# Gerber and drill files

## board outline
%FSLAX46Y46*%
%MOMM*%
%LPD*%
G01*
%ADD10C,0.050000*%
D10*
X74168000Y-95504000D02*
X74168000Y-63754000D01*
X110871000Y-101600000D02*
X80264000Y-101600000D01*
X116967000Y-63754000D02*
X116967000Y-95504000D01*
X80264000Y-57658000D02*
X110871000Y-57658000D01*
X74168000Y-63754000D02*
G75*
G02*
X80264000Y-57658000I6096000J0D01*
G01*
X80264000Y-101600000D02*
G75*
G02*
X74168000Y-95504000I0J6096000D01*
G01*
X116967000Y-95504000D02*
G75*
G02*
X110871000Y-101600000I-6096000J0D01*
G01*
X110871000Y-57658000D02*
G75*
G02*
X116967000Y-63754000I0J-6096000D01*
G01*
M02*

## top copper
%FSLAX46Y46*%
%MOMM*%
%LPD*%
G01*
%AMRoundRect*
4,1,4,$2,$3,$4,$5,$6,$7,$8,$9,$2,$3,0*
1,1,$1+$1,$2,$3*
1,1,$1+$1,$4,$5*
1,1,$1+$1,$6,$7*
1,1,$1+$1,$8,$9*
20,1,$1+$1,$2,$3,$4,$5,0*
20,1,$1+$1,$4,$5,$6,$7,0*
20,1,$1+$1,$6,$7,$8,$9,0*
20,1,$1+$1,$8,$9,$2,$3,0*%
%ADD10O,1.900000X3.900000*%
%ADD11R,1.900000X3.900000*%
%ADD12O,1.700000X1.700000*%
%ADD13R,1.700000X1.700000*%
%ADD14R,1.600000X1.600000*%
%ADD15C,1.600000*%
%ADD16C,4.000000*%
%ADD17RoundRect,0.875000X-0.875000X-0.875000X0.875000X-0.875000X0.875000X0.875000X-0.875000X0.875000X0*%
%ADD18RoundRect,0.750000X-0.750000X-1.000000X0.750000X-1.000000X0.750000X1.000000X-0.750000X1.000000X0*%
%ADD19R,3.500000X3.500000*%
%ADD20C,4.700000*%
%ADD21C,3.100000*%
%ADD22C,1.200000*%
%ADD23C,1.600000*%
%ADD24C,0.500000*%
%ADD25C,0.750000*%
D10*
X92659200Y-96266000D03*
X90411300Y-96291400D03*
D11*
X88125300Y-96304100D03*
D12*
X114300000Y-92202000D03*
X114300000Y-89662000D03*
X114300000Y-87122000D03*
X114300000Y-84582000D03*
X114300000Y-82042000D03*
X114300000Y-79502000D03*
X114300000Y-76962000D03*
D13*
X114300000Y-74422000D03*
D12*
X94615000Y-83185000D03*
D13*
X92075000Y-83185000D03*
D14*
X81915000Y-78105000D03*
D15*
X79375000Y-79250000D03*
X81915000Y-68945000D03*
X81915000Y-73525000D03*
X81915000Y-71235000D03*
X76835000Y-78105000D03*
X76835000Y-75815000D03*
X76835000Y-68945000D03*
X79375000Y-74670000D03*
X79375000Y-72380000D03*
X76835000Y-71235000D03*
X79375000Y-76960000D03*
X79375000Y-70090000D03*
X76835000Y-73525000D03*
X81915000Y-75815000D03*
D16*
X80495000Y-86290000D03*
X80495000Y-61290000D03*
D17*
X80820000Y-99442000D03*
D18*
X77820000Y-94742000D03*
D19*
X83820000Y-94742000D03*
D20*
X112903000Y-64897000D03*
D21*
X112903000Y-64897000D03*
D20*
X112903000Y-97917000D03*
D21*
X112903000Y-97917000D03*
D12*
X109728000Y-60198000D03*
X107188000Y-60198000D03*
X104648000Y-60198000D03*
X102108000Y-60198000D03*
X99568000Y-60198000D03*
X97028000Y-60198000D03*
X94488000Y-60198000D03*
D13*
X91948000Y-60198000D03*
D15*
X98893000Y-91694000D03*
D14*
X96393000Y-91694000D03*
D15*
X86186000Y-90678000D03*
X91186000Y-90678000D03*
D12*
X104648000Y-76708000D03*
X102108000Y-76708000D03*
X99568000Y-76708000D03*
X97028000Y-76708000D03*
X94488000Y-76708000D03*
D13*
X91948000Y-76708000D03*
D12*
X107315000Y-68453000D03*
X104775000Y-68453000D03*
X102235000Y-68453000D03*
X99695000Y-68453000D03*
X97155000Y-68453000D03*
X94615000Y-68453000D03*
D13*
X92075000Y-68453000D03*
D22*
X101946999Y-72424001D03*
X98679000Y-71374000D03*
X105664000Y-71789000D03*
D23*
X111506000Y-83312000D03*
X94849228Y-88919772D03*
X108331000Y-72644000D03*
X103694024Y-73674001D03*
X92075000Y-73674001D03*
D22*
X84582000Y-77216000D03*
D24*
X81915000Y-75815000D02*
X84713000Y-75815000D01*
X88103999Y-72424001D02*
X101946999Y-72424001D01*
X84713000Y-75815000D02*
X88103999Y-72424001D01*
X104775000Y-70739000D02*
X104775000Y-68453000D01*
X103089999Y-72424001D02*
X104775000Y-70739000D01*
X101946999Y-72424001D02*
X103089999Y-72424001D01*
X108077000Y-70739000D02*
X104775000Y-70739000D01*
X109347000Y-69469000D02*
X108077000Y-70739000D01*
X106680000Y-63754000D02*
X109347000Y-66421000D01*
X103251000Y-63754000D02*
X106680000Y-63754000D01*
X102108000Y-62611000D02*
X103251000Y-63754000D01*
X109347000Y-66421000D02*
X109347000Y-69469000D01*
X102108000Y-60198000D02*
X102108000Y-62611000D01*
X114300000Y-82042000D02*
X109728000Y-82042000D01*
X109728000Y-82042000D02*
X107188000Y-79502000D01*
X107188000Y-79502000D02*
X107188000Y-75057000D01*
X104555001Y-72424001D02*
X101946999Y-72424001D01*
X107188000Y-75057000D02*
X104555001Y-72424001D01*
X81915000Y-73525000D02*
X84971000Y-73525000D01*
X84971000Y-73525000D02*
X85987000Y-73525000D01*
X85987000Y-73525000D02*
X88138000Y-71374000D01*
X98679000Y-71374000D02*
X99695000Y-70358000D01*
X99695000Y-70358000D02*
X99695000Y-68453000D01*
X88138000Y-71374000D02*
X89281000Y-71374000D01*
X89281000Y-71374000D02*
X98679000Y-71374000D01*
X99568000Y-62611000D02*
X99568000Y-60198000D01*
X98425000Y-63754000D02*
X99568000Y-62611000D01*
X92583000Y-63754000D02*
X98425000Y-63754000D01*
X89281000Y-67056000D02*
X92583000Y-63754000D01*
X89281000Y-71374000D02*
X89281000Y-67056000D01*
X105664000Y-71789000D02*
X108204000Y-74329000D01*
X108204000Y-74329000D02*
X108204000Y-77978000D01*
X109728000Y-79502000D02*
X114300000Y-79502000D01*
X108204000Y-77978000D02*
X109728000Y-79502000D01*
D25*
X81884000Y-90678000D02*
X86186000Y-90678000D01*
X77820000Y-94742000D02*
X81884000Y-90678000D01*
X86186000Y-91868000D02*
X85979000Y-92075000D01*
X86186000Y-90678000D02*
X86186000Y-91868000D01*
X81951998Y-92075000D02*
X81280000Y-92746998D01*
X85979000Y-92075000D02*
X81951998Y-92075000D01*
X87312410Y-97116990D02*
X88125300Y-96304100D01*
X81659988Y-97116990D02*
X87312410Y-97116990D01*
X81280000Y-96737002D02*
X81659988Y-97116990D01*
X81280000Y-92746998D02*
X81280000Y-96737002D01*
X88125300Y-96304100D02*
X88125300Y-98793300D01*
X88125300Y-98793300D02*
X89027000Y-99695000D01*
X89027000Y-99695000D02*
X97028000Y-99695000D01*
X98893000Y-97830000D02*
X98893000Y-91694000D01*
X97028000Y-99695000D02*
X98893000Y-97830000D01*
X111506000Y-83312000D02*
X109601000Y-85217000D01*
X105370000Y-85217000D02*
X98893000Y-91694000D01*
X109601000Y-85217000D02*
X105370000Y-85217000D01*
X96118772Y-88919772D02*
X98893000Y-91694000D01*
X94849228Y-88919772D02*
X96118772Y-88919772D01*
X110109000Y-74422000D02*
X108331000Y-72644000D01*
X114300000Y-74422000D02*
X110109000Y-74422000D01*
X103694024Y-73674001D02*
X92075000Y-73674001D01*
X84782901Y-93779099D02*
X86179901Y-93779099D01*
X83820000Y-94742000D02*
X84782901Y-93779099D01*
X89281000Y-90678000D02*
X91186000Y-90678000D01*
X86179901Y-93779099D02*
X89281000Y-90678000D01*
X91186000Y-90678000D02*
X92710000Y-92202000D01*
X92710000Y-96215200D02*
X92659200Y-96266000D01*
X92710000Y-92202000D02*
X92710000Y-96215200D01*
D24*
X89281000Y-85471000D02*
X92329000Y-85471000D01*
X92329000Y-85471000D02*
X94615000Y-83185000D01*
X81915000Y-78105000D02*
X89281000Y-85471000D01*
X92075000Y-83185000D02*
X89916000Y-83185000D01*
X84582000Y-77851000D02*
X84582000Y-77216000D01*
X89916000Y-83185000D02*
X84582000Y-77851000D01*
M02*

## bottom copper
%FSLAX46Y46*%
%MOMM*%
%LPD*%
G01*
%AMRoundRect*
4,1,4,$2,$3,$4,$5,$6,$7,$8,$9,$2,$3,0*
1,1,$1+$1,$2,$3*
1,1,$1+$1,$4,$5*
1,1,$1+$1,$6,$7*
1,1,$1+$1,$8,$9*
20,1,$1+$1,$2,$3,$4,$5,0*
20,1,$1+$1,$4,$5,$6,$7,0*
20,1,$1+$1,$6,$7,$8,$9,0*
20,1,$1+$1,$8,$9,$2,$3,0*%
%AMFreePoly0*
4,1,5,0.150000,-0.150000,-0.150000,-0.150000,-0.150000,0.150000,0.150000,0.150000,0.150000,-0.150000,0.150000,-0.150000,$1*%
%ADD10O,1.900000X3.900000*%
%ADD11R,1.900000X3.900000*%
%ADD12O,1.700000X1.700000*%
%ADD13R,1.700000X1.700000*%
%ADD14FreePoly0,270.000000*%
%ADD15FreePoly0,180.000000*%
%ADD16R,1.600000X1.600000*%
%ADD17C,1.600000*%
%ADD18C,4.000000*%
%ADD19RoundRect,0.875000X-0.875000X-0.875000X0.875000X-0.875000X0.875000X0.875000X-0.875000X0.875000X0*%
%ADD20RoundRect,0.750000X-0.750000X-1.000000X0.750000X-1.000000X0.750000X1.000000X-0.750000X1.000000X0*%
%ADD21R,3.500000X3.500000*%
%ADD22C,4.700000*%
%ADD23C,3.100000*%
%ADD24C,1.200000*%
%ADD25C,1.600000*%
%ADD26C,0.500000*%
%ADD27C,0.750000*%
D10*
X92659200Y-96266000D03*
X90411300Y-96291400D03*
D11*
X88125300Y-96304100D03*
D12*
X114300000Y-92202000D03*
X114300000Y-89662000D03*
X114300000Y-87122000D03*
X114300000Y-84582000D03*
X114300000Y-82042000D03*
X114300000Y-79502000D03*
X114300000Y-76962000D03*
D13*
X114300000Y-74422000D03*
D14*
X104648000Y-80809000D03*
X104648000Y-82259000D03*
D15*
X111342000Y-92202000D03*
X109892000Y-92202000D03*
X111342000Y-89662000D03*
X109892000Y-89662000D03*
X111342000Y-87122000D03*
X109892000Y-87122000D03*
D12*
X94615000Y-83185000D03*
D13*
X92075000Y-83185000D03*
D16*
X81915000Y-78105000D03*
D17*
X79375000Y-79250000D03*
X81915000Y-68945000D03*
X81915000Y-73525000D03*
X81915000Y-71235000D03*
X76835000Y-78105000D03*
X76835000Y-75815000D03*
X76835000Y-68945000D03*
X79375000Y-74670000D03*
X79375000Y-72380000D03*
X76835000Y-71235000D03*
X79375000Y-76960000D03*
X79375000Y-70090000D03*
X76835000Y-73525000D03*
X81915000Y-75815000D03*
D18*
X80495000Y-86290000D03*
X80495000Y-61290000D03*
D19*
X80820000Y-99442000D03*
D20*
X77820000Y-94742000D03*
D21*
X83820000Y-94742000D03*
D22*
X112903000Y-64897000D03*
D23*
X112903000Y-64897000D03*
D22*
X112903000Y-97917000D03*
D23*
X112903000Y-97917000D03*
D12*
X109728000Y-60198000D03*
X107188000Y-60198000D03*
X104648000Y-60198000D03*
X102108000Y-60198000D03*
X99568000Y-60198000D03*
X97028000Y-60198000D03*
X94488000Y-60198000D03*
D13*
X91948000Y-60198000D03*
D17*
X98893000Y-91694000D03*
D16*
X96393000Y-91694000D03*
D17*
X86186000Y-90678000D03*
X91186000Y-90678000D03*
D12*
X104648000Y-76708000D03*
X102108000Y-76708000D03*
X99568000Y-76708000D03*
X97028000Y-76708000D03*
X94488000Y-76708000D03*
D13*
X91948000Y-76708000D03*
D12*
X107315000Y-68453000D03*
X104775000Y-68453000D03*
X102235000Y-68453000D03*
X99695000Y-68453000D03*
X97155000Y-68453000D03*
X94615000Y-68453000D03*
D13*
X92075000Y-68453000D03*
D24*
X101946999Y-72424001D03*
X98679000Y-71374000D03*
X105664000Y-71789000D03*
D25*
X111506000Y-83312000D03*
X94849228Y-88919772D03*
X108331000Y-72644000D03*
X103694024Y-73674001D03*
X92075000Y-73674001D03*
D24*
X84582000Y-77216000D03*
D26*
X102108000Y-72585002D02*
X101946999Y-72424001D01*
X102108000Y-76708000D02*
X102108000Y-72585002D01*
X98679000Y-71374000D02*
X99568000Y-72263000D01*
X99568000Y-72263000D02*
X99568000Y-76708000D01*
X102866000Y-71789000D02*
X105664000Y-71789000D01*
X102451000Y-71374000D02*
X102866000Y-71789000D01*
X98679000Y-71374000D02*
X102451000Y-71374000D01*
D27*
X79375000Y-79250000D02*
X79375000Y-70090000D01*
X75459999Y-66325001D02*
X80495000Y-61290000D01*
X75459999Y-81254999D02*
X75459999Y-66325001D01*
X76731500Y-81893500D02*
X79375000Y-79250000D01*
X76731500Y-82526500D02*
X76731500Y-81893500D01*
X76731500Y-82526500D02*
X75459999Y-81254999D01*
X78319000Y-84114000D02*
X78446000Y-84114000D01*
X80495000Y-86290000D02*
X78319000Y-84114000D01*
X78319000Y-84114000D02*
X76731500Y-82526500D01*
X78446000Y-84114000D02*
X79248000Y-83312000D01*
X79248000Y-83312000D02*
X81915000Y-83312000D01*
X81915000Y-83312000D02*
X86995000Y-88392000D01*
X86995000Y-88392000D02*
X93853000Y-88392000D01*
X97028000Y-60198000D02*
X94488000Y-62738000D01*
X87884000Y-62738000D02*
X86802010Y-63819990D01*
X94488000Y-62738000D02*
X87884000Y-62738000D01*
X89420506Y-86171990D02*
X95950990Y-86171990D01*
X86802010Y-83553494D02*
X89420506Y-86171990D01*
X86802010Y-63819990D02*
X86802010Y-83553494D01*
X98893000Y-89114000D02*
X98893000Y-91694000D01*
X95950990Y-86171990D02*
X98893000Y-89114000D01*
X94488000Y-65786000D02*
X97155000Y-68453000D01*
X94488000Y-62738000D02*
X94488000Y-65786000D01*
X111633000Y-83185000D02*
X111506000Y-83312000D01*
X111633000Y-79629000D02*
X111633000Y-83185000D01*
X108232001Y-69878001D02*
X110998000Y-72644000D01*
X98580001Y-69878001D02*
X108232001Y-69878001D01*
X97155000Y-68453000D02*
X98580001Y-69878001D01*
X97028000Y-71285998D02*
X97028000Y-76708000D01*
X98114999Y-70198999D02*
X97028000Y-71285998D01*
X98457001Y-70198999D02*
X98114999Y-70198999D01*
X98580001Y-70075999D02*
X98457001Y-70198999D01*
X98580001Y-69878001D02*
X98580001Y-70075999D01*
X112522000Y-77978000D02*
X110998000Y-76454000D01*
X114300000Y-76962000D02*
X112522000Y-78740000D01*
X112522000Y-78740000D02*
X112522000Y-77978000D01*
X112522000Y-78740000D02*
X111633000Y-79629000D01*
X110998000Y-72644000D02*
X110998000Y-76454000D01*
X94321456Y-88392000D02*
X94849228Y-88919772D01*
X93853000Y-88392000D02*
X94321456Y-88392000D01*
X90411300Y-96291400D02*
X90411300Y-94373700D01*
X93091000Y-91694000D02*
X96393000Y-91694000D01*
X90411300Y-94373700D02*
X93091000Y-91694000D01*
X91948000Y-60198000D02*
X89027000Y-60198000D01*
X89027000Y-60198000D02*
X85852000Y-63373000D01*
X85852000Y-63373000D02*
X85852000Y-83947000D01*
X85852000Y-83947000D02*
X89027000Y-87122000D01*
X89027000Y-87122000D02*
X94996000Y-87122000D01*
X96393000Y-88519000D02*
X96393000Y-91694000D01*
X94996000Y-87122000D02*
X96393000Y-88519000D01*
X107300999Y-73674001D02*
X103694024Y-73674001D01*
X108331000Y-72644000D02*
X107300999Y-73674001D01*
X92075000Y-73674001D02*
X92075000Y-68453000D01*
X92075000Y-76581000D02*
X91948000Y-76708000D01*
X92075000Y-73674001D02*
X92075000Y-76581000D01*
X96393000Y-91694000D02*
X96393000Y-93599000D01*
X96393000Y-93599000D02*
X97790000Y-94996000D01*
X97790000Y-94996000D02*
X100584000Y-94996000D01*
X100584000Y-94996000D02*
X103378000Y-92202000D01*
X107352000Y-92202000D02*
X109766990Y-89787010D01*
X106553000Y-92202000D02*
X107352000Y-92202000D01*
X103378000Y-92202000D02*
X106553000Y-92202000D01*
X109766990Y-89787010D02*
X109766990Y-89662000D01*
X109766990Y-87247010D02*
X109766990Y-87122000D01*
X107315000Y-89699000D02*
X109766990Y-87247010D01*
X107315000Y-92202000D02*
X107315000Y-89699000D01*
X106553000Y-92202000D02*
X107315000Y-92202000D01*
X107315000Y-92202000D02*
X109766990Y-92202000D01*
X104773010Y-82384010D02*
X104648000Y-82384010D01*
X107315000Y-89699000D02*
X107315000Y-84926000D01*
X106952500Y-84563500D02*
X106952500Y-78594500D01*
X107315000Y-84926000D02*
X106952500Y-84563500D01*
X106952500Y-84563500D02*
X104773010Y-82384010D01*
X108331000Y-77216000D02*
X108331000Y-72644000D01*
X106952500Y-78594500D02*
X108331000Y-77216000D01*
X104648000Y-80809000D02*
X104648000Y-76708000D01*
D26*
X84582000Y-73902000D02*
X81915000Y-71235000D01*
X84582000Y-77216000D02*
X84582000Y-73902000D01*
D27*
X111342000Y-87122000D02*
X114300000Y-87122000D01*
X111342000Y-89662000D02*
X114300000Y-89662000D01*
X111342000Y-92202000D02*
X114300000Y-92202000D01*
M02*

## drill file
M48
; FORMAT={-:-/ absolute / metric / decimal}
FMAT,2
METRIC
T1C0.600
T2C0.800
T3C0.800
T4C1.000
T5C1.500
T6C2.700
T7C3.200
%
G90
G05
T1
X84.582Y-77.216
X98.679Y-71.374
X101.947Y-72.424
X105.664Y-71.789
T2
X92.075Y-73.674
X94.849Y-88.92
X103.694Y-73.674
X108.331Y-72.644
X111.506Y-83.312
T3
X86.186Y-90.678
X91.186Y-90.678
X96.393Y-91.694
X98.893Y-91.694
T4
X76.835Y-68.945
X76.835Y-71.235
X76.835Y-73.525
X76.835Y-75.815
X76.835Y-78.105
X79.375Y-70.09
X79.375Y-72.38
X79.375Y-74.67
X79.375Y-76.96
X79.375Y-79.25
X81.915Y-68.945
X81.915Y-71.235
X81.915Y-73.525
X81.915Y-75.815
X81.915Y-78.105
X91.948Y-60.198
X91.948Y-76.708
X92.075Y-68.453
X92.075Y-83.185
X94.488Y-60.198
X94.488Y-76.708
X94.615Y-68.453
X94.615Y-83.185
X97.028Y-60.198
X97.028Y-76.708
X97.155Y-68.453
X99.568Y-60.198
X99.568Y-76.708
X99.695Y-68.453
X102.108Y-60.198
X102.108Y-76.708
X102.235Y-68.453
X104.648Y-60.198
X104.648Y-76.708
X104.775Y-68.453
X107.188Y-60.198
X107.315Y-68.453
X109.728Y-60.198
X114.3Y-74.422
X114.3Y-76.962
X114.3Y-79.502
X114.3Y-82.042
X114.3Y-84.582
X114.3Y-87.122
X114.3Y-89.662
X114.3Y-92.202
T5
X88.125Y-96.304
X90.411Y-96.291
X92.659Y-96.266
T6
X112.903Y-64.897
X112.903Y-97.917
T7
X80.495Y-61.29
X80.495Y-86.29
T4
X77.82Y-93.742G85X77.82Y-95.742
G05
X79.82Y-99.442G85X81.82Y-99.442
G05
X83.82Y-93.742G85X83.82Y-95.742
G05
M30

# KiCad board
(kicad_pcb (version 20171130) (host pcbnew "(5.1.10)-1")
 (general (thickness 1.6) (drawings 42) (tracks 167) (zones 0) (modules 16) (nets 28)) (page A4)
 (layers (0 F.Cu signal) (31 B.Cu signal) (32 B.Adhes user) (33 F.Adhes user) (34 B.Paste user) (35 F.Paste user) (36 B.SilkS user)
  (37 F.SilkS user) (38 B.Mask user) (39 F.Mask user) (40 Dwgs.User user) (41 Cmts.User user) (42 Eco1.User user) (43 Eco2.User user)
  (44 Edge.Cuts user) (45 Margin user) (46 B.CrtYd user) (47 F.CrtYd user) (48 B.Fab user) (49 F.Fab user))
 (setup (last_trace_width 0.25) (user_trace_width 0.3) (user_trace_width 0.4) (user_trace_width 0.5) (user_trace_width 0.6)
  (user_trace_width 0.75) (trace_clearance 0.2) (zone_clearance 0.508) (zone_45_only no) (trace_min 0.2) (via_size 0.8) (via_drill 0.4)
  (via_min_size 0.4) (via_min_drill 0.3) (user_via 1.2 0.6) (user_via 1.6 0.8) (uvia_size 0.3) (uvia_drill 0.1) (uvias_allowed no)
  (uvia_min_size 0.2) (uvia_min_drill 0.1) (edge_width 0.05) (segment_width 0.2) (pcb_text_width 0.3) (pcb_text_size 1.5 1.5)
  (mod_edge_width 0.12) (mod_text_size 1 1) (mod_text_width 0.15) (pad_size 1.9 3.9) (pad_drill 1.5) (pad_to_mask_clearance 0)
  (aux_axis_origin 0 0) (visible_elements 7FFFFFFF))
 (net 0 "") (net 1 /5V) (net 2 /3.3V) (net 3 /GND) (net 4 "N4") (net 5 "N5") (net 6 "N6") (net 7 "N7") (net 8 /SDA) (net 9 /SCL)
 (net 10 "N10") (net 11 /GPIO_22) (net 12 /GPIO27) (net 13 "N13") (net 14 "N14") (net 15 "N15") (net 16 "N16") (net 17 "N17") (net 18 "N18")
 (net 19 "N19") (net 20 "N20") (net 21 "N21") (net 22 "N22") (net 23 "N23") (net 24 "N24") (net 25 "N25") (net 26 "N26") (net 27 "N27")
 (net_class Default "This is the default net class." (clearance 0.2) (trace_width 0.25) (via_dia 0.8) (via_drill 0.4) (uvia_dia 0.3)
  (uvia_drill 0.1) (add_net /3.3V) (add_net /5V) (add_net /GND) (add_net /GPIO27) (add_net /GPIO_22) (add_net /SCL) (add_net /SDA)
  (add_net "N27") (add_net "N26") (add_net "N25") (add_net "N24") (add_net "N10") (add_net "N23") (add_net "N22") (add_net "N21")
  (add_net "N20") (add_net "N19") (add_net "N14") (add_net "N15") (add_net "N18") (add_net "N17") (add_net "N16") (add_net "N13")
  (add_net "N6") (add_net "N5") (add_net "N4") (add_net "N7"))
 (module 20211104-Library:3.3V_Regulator (layer F.Cu) (at 84.963 96.266)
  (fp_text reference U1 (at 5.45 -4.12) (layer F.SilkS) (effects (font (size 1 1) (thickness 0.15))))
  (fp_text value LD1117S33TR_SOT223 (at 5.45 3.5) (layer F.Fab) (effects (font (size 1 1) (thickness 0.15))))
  (pad 3 thru_hole oval (at 7.6962 0) (size 1.9 3.9) (drill 1.5) (layers *.Cu *.Mask) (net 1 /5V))
  (pad 2 thru_hole oval (at 5.4483 0.0254) (size 1.9 3.9) (drill 1.5) (layers *.Cu *.Mask) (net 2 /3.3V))
  (pad 1 thru_hole rect (at 3.1623 0.0381) (size 1.9 3.9) (drill 1.5) (layers *.Cu *.Mask) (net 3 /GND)))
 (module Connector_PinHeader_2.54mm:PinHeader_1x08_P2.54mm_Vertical (layer F.Cu) (at 114.3 74.422)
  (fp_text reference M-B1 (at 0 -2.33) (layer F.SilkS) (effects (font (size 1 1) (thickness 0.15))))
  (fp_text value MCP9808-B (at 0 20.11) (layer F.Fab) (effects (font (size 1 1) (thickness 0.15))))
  (pad 8 thru_hole oval (at 0 17.78) (size 1.7 1.7) (drill 1) (layers *.Cu *.Mask) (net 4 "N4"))
  (pad 7 thru_hole oval (at 0 15.24) (size 1.7 1.7) (drill 1) (layers *.Cu *.Mask) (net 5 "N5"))
  (pad 6 thru_hole oval (at 0 12.7) (size 1.7 1.7) (drill 1) (layers *.Cu *.Mask) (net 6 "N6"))
  (pad 5 thru_hole oval (at 0 10.16) (size 1.7 1.7) (drill 1) (layers *.Cu *.Mask) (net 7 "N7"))
  (pad 4 thru_hole oval (at 0 7.62) (size 1.7 1.7) (drill 1) (layers *.Cu *.Mask) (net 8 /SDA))
  (pad 3 thru_hole oval (at 0 5.08) (size 1.7 1.7) (drill 1) (layers *.Cu *.Mask) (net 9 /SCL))
  (pad 2 thru_hole oval (at 0 2.54) (size 1.7 1.7) (drill 1) (layers *.Cu *.Mask) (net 3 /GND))
  (pad 1 thru_hole rect (at 0 0) (size 1.7 1.7) (drill 1) (layers *.Cu *.Mask) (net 2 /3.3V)))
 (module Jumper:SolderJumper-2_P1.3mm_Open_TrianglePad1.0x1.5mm (layer B.Cu) (at 104.648 81.534 270)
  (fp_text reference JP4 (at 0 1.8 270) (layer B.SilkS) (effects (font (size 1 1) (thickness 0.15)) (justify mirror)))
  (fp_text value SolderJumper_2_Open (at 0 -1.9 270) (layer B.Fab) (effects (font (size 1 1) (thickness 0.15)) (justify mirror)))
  (pad 1 smd custom (at -0.725 0 270) (size 0.3 0.3) (layers B.Cu B.Mask) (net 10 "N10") (zone_connect 2)
   (options (clearance outline) (anchor rect)) (primitives))
  (pad 2 smd custom (at 0.725 0 270) (size 0.3 0.3) (layers B.Cu B.Mask) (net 2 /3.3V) (zone_connect 2)
   (options (clearance outline) (anchor rect)) (primitives)))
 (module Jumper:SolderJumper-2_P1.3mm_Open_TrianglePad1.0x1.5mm (layer B.Cu) (at 110.617 92.202 180)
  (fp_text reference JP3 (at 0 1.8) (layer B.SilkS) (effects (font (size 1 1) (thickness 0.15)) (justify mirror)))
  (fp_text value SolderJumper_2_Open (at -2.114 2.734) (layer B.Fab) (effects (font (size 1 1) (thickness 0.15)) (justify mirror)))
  (pad 1 smd custom (at -0.725 0 180) (size 0.3 0.3) (layers B.Cu B.Mask) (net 4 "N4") (zone_connect 2)
   (options (clearance outline) (anchor rect)) (primitives))
  (pad 2 smd custom (at 0.725 0 180) (size 0.3 0.3) (layers B.Cu B.Mask) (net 2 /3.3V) (zone_connect 2)
   (options (clearance outline) (anchor rect)) (primitives)))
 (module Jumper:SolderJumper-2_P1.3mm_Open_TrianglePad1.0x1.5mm (layer B.Cu) (at 110.617 89.662 180)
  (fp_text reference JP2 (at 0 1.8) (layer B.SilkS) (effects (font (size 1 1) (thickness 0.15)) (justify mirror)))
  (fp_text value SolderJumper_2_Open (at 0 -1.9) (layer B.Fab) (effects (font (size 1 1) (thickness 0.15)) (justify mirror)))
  (pad 1 smd custom (at -0.725 0 180) (size 0.3 0.3) (layers B.Cu B.Mask) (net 5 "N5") (zone_connect 2)
   (options (clearance outline) (anchor rect)) (primitives))
  (pad 2 smd custom (at 0.725 0 180) (size 0.3 0.3) (layers B.Cu B.Mask) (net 2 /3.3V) (zone_connect 2)
   (options (clearance outline) (anchor rect)) (primitives)))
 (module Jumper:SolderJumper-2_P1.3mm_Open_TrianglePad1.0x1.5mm (layer B.Cu) (at 110.617 87.122 180)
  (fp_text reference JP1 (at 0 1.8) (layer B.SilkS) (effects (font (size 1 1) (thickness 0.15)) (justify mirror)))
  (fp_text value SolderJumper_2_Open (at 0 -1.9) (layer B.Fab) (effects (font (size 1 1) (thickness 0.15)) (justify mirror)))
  (pad 1 smd custom (at -0.725 0 180) (size 0.3 0.3) (layers B.Cu B.Mask) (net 6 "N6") (zone_connect 2)
   (options (clearance outline) (anchor rect)) (primitives))
  (pad 2 smd custom (at 0.725 0 180) (size 0.3 0.3) (layers B.Cu B.Mask) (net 2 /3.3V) (zone_connect 2)
   (options (clearance outline) (anchor rect)) (primitives)))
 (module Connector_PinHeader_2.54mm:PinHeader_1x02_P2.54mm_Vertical (layer F.Cu) (at 92.075 83.185 90)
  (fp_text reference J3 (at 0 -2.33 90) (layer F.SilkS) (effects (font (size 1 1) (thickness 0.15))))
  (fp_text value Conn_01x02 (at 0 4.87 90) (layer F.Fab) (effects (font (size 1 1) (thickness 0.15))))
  (pad 2 thru_hole oval (at 0 2.54 90) (size 1.7 1.7) (drill 1) (layers *.Cu *.Mask) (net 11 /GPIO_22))
  (pad 1 thru_hole rect (at 0 0 90) (size 1.7 1.7) (drill 1) (layers *.Cu *.Mask) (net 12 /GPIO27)))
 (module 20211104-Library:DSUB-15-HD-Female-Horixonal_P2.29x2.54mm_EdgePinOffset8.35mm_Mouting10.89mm (layer F.Cu) (at 81.915 78.105 270)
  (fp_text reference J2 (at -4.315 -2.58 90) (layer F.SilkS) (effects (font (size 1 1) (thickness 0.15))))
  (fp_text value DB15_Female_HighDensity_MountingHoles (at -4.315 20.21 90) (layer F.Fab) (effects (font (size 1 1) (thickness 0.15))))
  (pad 1 thru_hole rect (at 0 0 270) (size 1.6 1.6) (drill 1) (layers *.Cu *.Mask) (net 11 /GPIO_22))
  (pad 6 thru_hole circle (at 1.145 2.54 270) (size 1.6 1.6) (drill 1) (layers *.Cu *.Mask) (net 3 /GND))
  (pad 5 thru_hole circle (at -9.16 0 270) (size 1.6 1.6) (drill 1) (layers *.Cu *.Mask) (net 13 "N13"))
  (pad 3 thru_hole circle (at -4.58 0 270) (size 1.6 1.6) (drill 1) (layers *.Cu *.Mask) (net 9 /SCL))
  (pad 4 thru_hole circle (at -6.87 0 270) (size 1.6 1.6) (drill 1) (layers *.Cu *.Mask) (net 12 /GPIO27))
  (pad 11 thru_hole circle (at 0 5.08 270) (size 1.6 1.6) (drill 1) (layers *.Cu *.Mask) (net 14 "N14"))
  (pad 12 thru_hole circle (at -2.29 5.08 270) (size 1.6 1.6) (drill 1) (layers *.Cu *.Mask) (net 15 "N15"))
  (pad 15 thru_hole circle (at -9.16 5.08 270) (size 1.6 1.6) (drill 1) (layers *.Cu *.Mask) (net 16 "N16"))
  (pad 8 thru_hole circle (at -3.435 2.54 270) (size 1.6 1.6) (drill 1) (layers *.Cu *.Mask) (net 3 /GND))
  (pad 9 thru_hole circle (at -5.725 2.54 270) (size 1.6 1.6) (drill 1) (layers *.Cu *.Mask) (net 3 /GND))
  (pad 14 thru_hole circle (at -6.87 5.08 270) (size 1.6 1.6) (drill 1) (layers *.Cu *.Mask) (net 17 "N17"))
  (pad 7 thru_hole circle (at -1.145 2.54 270) (size 1.6 1.6) (drill 1) (layers *.Cu *.Mask) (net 3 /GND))
  (pad 10 thru_hole circle (at -8.015 2.54 270) (size 1.6 1.6) (drill 1) (layers *.Cu *.Mask) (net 3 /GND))
  (pad 13 thru_hole circle (at -4.58 5.08 270) (size 1.6 1.6) (drill 1) (layers *.Cu *.Mask) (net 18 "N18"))
  (pad 2 thru_hole circle (at -2.29 0 270) (size 1.6 1.6) (drill 1) (layers *.Cu *.Mask) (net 8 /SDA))
  (pad 0 thru_hole circle (at 8.185 1.42 270) (size 4 4) (drill 3.2) (layers *.Cu *.Mask) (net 3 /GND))
  (pad 0 thru_hole circle (at -16.815 1.42 270) (size 4 4) (drill 3.2) (layers *.Cu *.Mask) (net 3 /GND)))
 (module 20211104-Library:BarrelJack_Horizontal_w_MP (layer F.Cu) (at 83.82 94.742)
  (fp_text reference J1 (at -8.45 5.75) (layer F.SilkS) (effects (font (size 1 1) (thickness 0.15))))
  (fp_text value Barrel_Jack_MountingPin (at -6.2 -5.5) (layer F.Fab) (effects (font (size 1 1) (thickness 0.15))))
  (pad MP thru_hole roundrect (at -3 4.7) (size 3.5 3.5) (drill oval 3 1) (layers *.Cu *.Mask) (roundrect_rratio 0.25) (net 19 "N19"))
  (pad 2 thru_hole roundrect (at -6 0) (size 3 3.5) (drill oval 1 3) (layers *.Cu *.Mask) (roundrect_rratio 0.25) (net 3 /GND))
  (pad 1 thru_hole rect (at 0 0) (size 3.5 3.5) (drill oval 1 3) (layers *.Cu *.Mask) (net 1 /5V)))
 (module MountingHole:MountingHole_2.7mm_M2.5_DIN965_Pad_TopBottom (layer F.Cu) (at 112.903 64.897)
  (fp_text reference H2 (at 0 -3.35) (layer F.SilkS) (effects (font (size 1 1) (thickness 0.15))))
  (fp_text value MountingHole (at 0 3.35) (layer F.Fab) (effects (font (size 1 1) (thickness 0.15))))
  (pad 1 connect circle (at 0 0) (size 4.7 4.7) (layers B.Cu B.Mask))
  (pad 1 connect circle (at 0 0) (size 4.7 4.7) (layers F.Cu F.Mask))
  (pad 1 thru_hole circle (at 0 0) (size 3.1 3.1) (drill 2.7) (layers *.Cu *.Mask)))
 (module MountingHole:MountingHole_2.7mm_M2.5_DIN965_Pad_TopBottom (layer F.Cu) (at 112.903 97.917)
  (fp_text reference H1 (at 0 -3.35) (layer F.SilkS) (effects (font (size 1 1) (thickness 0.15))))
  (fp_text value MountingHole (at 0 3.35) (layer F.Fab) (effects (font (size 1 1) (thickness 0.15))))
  (pad 1 connect circle (at 0 0) (size 4.7 4.7) (layers B.Cu B.Mask))
  (pad 1 connect circle (at 0 0) (size 4.7 4.7) (layers F.Cu F.Mask))
  (pad 1 thru_hole circle (at 0 0) (size 3.1 3.1) (drill 2.7) (layers *.Cu *.Mask)))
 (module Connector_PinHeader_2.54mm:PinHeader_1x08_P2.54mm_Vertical (layer F.Cu) (at 91.948 60.198 90)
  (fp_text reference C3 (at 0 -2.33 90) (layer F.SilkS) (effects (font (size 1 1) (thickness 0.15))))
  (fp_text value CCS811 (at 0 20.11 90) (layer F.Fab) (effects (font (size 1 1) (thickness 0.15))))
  (pad 8 thru_hole oval (at 0 17.78 90) (size 1.7 1.7) (drill 1) (layers *.Cu *.Mask) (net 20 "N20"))
  (pad 7 thru_hole oval (at 0 15.24 90) (size 1.7 1.7) (drill 1) (layers *.Cu *.Mask) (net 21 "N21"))
  (pad 6 thru_hole oval (at 0 12.7 90) (size 1.7 1.7) (drill 1) (layers *.Cu *.Mask) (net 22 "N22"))
  (pad 5 thru_hole oval (at 0 10.16 90) (size 1.7 1.7) (drill 1) (layers *.Cu *.Mask) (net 8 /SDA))
  (pad 4 thru_hole oval (at 0 7.62 90) (size 1.7 1.7) (drill 1) (layers *.Cu *.Mask) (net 9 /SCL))
  (pad 3 thru_hole oval (at 0 5.08 90) (size 1.7 1.7) (drill 1) (layers *.Cu *.Mask) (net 3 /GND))
  (pad 2 thru_hole oval (at 0 2.54 90) (size 1.7 1.7) (drill 1) (layers *.Cu *.Mask) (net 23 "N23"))
  (pad 1 thru_hole rect (at 0 0 90) (size 1.7 1.7) (drill 1) (layers *.Cu *.Mask) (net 2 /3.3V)))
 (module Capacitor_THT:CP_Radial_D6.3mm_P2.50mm (layer F.Cu) (at 96.393 91.694)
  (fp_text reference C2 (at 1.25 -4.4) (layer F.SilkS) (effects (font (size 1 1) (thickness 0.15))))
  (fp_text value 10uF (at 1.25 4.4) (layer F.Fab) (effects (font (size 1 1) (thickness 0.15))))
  (pad 2 thru_hole circle (at 2.5 0) (size 1.6 1.6) (drill 0.8) (layers *.Cu *.Mask) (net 3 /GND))
  (pad 1 thru_hole rect (at 0 0) (size 1.6 1.6) (drill 0.8) (layers *.Cu *.Mask) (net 2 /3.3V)))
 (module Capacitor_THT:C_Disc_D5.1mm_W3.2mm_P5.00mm (layer F.Cu) (at 91.186 90.678 180)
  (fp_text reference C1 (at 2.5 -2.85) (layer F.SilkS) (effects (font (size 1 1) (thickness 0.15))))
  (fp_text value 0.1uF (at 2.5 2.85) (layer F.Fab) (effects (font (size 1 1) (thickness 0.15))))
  (pad 2 thru_hole circle (at 5 0 180) (size 1.6 1.6) (drill 0.8) (layers *.Cu *.Mask) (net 3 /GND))
  (pad 1 thru_hole circle (at 0 0 180) (size 1.6 1.6) (drill 0.8) (layers *.Cu *.Mask) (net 1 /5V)))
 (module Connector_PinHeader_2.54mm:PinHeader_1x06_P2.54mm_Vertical (layer F.Cu) (at 91.948 76.708 90)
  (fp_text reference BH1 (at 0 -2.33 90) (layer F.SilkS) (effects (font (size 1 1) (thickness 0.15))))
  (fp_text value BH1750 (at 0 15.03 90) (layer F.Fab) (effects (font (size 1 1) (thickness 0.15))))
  (pad 6 thru_hole oval (at 0 12.7 90) (size 1.7 1.7) (drill 1) (layers *.Cu *.Mask) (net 10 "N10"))
  (pad 5 thru_hole oval (at 0 10.16 90) (size 1.7 1.7) (drill 1) (layers *.Cu *.Mask) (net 8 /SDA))
  (pad 4 thru_hole oval (at 0 7.62 90) (size 1.7 1.7) (drill 1) (layers *.Cu *.Mask) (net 9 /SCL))
  (pad 3 thru_hole oval (at 0 5.08 90) (size 1.7 1.7) (drill 1) (layers *.Cu *.Mask) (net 3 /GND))
  (pad 2 thru_hole oval (at 0 2.54 90) (size 1.7 1.7) (drill 1) (layers *.Cu *.Mask) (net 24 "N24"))
  (pad 1 thru_hole rect (at 0 0 90) (size 1.7 1.7) (drill 1) (layers *.Cu *.Mask) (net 2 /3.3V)))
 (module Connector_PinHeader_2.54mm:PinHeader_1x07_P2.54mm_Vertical (layer F.Cu) (at 92.075 68.453 90)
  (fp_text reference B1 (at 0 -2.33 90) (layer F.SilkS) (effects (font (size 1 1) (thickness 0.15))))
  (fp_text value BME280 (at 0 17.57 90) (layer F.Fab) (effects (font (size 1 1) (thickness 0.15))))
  (pad 7 thru_hole oval (at 0 15.24 90) (size 1.7 1.7) (drill 1) (layers *.Cu *.Mask) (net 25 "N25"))
  (pad 6 thru_hole oval (at 0 12.7 90) (size 1.7 1.7) (drill 1) (layers *.Cu *.Mask) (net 8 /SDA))
  (pad 5 thru_hole oval (at 0 10.16 90) (size 1.7 1.7) (drill 1) (layers *.Cu *.Mask) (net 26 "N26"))
  (pad 4 thru_hole oval (at 0 7.62 90) (size 1.7 1.7) (drill 1) (layers *.Cu *.Mask) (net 9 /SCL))
  (pad 3 thru_hole oval (at 0 5.08 90) (size 1.7 1.7) (drill 1) (layers *.Cu *.Mask) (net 3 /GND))
  (pad 2 thru_hole oval (at 0 2.54 90) (size 1.7 1.7) (drill 1) (layers *.Cu *.Mask) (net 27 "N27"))
  (pad 1 thru_hole rect (at 0 0 90) (size 1.7 1.7) (drill 1) (layers *.Cu *.Mask) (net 2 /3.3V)))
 (gr_line (start 74.168 95.504) (end 74.168 63.754) (layer Edge.Cuts) (width 0.05))
 (gr_line (start 110.871 101.6) (end 80.264 101.6) (layer Edge.Cuts) (width 0.05))
 (gr_line (start 116.967 63.754) (end 116.967 95.504) (layer Edge.Cuts) (width 0.05))
 (gr_line (start 80.264 57.658) (end 110.871 57.658) (layer Edge.Cuts) (width 0.05))
 (gr_arc (start 80.264 63.754) (end 80.264 57.658) (angle -90) (layer Edge.Cuts) (width 0.05))
 (gr_arc (start 80.264 95.504) (end 74.168 95.504) (angle -90) (layer Edge.Cuts) (width 0.05))
 (gr_arc (start 110.871 95.504) (end 110.871 101.6) (angle -90) (layer Edge.Cuts) (width 0.05))
 (gr_arc (start 110.871 63.754) (end 116.967 63.754) (angle -90) (layer Edge.Cuts) (width 0.05))
 (segment (start 81.915 75.815) (end 84.713 75.815) (width 0.5) (layer F.Cu) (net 8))
 (segment (start 88.103999 72.424001) (end 101.946999 72.424001) (width 0.5) (layer F.Cu) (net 8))
 (segment (start 84.713 75.815) (end 88.103999 72.424001) (width 0.5) (layer F.Cu) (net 8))
 (segment (start 104.775 70.739) (end 104.775 68.453) (width 0.5) (layer F.Cu) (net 8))
 (segment (start 103.089999 72.424001) (end 104.775 70.739) (width 0.5) (layer F.Cu) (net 8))
 (segment (start 101.946999 72.424001) (end 103.089999 72.424001) (width 0.5) (layer F.Cu) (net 8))
 (via (at 101.946999 72.424001) (size 1.2) (drill 0.6) (layers F.Cu B.Cu) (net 8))
 (segment (start 102.108 72.585002) (end 101.946999 72.424001) (width 0.5) (layer B.Cu) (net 8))
 (segment (start 102.108 76.708) (end 102.108 72.585002) (width 0.5) (layer B.Cu) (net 8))
 (segment (start 108.077 70.739) (end 104.775 70.739) (width 0.5) (layer F.Cu) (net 8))
 (segment (start 109.347 69.469) (end 108.077 70.739) (width 0.5) (layer F.Cu) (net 8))
 (segment (start 106.68 63.754) (end 109.347 66.421) (width 0.5) (layer F.Cu) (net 8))
 (segment (start 103.251 63.754) (end 106.68 63.754) (width 0.5) (layer F.Cu) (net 8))
 (segment (start 102.108 62.611) (end 103.251 63.754) (width 0.5) (layer F.Cu) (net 8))
 (segment (start 109.347 66.421) (end 109.347 69.469) (width 0.5) (layer F.Cu) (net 8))
 (segment (start 102.108 60.198) (end 102.108 62.611) (width 0.5) (layer F.Cu) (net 8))
 (segment (start 114.3 82.042) (end 109.728 82.042) (width 0.5) (layer F.Cu) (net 8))
 (segment (start 109.728 82.042) (end 107.188 79.502) (width 0.5) (layer F.Cu) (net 8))
 (segment (start 107.188 79.502) (end 107.188 75.057) (width 0.5) (layer F.Cu) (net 8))
 (segment (start 104.555001 72.424001) (end 101.946999 72.424001) (width 0.5) (layer F.Cu) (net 8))
 (segment (start 107.188 75.057) (end 104.555001 72.424001) (width 0.5) (layer F.Cu) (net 8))
 (segment (start 81.915 73.525) (end 84.971 73.525) (width 0.5) (layer F.Cu) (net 9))
 (segment (start 84.971 73.525) (end 85.987 73.525) (width 0.5) (layer F.Cu) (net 9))
 (via (at 98.679 71.374) (size 1.2) (drill 0.6) (layers F.Cu B.Cu) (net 9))
 (segment (start 85.987 73.525) (end 88.138 71.374) (width 0.5) (layer F.Cu) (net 9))
 (segment (start 98.679 71.374) (end 99.568 72.263) (width 0.5) (layer B.Cu) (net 9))
 (segment (start 99.568 72.263) (end 99.568 76.708) (width 0.5) (layer B.Cu) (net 9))
 (segment (start 98.679 71.374) (end 99.695 70.358) (width 0.5) (layer F.Cu) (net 9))
 (segment (start 99.695 70.358) (end 99.695 68.453) (width 0.5) (layer F.Cu) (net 9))
 (segment (start 88.138 71.374) (end 89.281 71.374) (width 0.5) (layer F.Cu) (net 9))
 (segment (start 89.281 71.374) (end 98.679 71.374) (width 0.5) (layer F.Cu) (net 9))
 (segment (start 99.568 62.611) (end 99.568 60.198) (width 0.5) (layer F.Cu) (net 9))
 (segment (start 98.425 63.754) (end 99.568 62.611) (width 0.5) (layer F.Cu) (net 9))
 (segment (start 92.583 63.754) (end 98.425 63.754) (width 0.5) (layer F.Cu) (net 9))
 (segment (start 89.281 67.056) (end 92.583 63.754) (width 0.5) (layer F.Cu) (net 9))
 (segment (start 89.281 71.374) (end 89.281 67.056) (width 0.5) (layer F.Cu) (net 9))
 (via (at 105.664 71.789) (size 1.2) (drill 0.6) (layers F.Cu B.Cu) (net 9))
 (segment (start 102.866 71.789) (end 105.664 71.789) (width 0.5) (layer B.Cu) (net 9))
 (segment (start 102.451 71.374) (end 102.866 71.789) (width 0.5) (layer B.Cu) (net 9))
 (segment (start 98.679 71.374) (end 102.451 71.374) (width 0.5) (layer B.Cu) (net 9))
 (segment (start 105.664 71.789) (end 108.204 74.329) (width 0.5) (layer F.Cu) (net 9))
 (segment (start 108.204 74.329) (end 108.204 77.978) (width 0.5) (layer F.Cu) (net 9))
 (segment (start 109.728 79.502) (end 114.3 79.502) (width 0.5) (layer F.Cu) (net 9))
 (segment (start 108.204 77.978) (end 109.728 79.502) (width 0.5) (layer F.Cu) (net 9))
 (segment (start 81.884 90.678) (end 86.186 90.678) (width 0.75) (layer F.Cu) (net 3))
 (segment (start 77.82 94.742) (end 81.884 90.678) (width 0.75) (layer F.Cu) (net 3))
 (segment (start 86.186 91.868) (end 85.979 92.075) (width 0.75) (layer F.Cu) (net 3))
 (segment (start 86.186 90.678) (end 86.186 91.868) (width 0.75) (layer F.Cu) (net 3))
 (segment (start 81.951998 92.075) (end 81.28 92.746998) (width 0.75) (layer F.Cu) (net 3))
 (segment (start 85.979 92.075) (end 81.951998 92.075) (width 0.75) (layer F.Cu) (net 3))
 (segment (start 87.31241 97.11699) (end 88.1253 96.3041) (width 0.75) (layer F.Cu) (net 3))
 (segment (start 81.659988 97.11699) (end 87.31241 97.11699) (width 0.75) (layer F.Cu) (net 3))
 (segment (start 81.28 96.737002) (end 81.659988 97.11699) (width 0.75) (layer F.Cu) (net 3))
 (segment (start 81.28 92.746998) (end 81.28 96.737002) (width 0.75) (layer F.Cu) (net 3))
 (segment (start 88.1253 96.3041) (end 88.1253 98.7933) (width 0.75) (layer F.Cu) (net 3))
 (segment (start 88.1253 98.7933) (end 89.027 99.695) (width 0.75) (layer F.Cu) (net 3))
 (segment (start 89.027 99.695) (end 97.028 99.695) (width 0.75) (layer F.Cu) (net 3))
 (segment (start 98.893 97.83) (end 98.893 91.694) (width 0.75) (layer F.Cu) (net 3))
 (segment (start 97.028 99.695) (end 98.893 97.83) (width 0.75) (layer F.Cu) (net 3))
 (segment (start 79.375 79.25) (end 79.375 70.09) (width 0.75) (layer B.Cu) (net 3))
 (segment (start 75.459999 66.325001) (end 80.495 61.29) (width 0.75) (layer B.Cu) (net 3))
 (segment (start 75.459999 81.254999) (end 75.459999 66.325001) (width 0.75) (layer B.Cu) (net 3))
 (segment (start 76.7315 81.8935) (end 79.375 79.25) (width 0.75) (layer B.Cu) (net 3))
 (segment (start 76.7315 82.5265) (end 76.7315 81.8935) (width 0.75) (layer B.Cu) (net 3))
 (segment (start 76.7315 82.5265) (end 75.459999 81.254999) (width 0.75) (layer B.Cu) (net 3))
 (segment (start 78.319 84.114) (end 78.446 84.114) (width 0.75) (layer B.Cu) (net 3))
 (segment (start 80.495 86.29) (end 78.319 84.114) (width 0.75) (layer B.Cu) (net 3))
 (segment (start 78.319 84.114) (end 76.7315 82.5265) (width 0.75) (layer B.Cu) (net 3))
 (segment (start 78.446 84.114) (end 79.248 83.312) (width 0.75) (layer B.Cu) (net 3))
 (segment (start 79.248 83.312) (end 81.915 83.312) (width 0.75) (layer B.Cu) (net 3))
 (segment (start 81.915 83.312) (end 86.995 88.392) (width 0.75) (layer B.Cu) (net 3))
 (segment (start 86.995 88.392) (end 93.853 88.392) (width 0.75) (layer B.Cu) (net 3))
 (segment (start 97.028 60.198) (end 94.488 62.738) (width 0.75) (layer B.Cu) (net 3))
 (segment (start 87.884 62.738) (end 86.80201 63.81999) (width 0.75) (layer B.Cu) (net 3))
 (segment (start 94.488 62.738) (end 87.884 62.738) (width 0.75) (layer B.Cu) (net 3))
 (segment (start 89.420506 86.17199) (end 95.95099 86.17199) (width 0.75) (layer B.Cu) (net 3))
 (segment (start 86.80201 83.553494) (end 89.420506 86.17199) (width 0.75) (layer B.Cu) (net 3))
 (segment (start 86.80201 63.81999) (end 86.80201 83.553494) (width 0.75) (layer B.Cu) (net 3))
 (segment (start 98.893 89.114) (end 98.893 91.694) (width 0.75) (layer B.Cu) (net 3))
 (segment (start 95.95099 86.17199) (end 98.893 89.114) (width 0.75) (layer B.Cu) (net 3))
 (segment (start 94.488 65.786) (end 97.155 68.453) (width 0.75) (layer B.Cu) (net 3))
 (segment (start 94.488 62.738) (end 94.488 65.786) (width 0.75) (layer B.Cu) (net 3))
 (via (at 111.506 83.312) (size 1.6) (drill 0.8) (layers F.Cu B.Cu) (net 3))
 (segment (start 111.633 83.185) (end 111.506 83.312) (width 0.75) (layer B.Cu) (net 3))
 (segment (start 111.633 79.629) (end 111.633 83.185) (width 0.75) (layer B.Cu) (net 3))
 (segment (start 111.506 83.312) (end 109.601 85.217) (width 0.75) (layer F.Cu) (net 3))
 (segment (start 105.37 85.217) (end 98.893 91.694) (width 0.75) (layer F.Cu) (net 3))
 (segment (start 109.601 85.217) (end 105.37 85.217) (width 0.75) (layer F.Cu) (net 3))
 (segment (start 108.232001 69.878001) (end 110.998 72.644) (width 0.75) (layer B.Cu) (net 3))
 (segment (start 98.580001 69.878001) (end 108.232001 69.878001) (width 0.75) (layer B.Cu) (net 3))
 (segment (start 97.155 68.453) (end 98.580001 69.878001) (width 0.75) (layer B.Cu) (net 3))
 (segment (start 97.028 71.285998) (end 97.028 76.708) (width 0.75) (layer B.Cu) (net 3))
 (segment (start 98.114999 70.198999) (end 97.028 71.285998) (width 0.75) (layer B.Cu) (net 3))
 (segment (start 98.457001 70.198999) (end 98.114999 70.198999) (width 0.75) (layer B.Cu) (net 3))
 (segment (start 98.580001 70.075999) (end 98.457001 70.198999) (width 0.75) (layer B.Cu) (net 3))
 (segment (start 98.580001 69.878001) (end 98.580001 70.075999) (width 0.75) (layer B.Cu) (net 3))
 (segment (start 112.522 77.978) (end 110.998 76.454) (width 0.75) (layer B.Cu) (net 3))
 (segment (start 114.3 76.962) (end 112.522 78.74) (width 0.75) (layer B.Cu) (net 3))
 (segment (start 112.522 78.74) (end 112.522 77.978) (width 0.75) (layer B.Cu) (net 3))
 (segment (start 112.522 78.74) (end 111.633 79.629) (width 0.75) (layer B.Cu) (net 3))
 (segment (start 110.998 72.644) (end 110.998 76.454) (width 0.75) (layer B.Cu) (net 3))
 (via (at 94.849228 88.919772) (size 1.6) (drill 0.8) (layers F.Cu B.Cu) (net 3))
 (segment (start 94.321456 88.392) (end 94.849228 88.919772) (width 0.75) (layer B.Cu) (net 3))
 (segment (start 93.853 88.392) (end 94.321456 88.392) (width 0.75) (layer B.Cu) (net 3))
 (segment (start 96.118772 88.919772) (end 98.893 91.694) (width 0.75) (layer F.Cu) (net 3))
 (segment (start 94.849228 88.919772) (end 96.118772 88.919772) (width 0.75) (layer F.Cu) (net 3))
 (segment (start 90.4113 96.2914) (end 90.4113 94.3737) (width 0.75) (layer B.Cu) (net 2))
 (segment (start 93.091 91.694) (end 96.393 91.694) (width 0.75) (layer B.Cu) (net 2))
 (segment (start 90.4113 94.3737) (end 93.091 91.694) (width 0.75) (layer B.Cu) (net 2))
 (segment (start 91.948 60.198) (end 89.027 60.198) (width 0.75) (layer B.Cu) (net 2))
 (segment (start 89.027 60.198) (end 85.852 63.373) (width 0.75) (layer B.Cu) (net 2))
 (segment (start 85.852 63.373) (end 85.852 83.947) (width 0.75) (layer B.Cu) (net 2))
 (segment (start 85.852 83.947) (end 89.027 87.122) (width 0.75) (layer B.Cu) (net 2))
 (segment (start 89.027 87.122) (end 94.996 87.122) (width 0.75) (layer B.Cu) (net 2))
 (segment (start 96.393 88.519) (end 96.393 91.694) (width 0.75) (layer B.Cu) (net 2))
 (segment (start 94.996 87.122) (end 96.393 88.519) (width 0.75) (layer B.Cu) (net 2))
 (via (at 108.331 72.644) (size 1.6) (drill 0.8) (layers F.Cu B.Cu) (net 2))
 (segment (start 110.109 74.422) (end 108.331 72.644) (width 0.75) (layer F.Cu) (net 2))
 (segment (start 114.3 74.422) (end 110.109 74.422) (width 0.75) (layer F.Cu) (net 2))
 (via (at 103.694024 73.674001) (size 1.6) (drill 0.8) (layers F.Cu B.Cu) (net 2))
 (segment (start 107.300999 73.674001) (end 103.694024 73.674001) (width 0.75) (layer B.Cu) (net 2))
 (segment (start 108.331 72.644) (end 107.300999 73.674001) (width 0.75) (layer B.Cu) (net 2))
 (via (at 92.075 73.674001) (size 1.6) (drill 0.8) (layers F.Cu B.Cu) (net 2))
 (segment (start 103.694024 73.674001) (end 92.075 73.674001) (width 0.75) (layer F.Cu) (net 2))
 (segment (start 92.075 73.674001) (end 92.075 68.453) (width 0.75) (layer B.Cu) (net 2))
 (segment (start 92.075 76.581) (end 91.948 76.708) (width 0.75) (layer B.Cu) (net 2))
 (segment (start 92.075 73.674001) (end 92.075 76.581) (width 0.75) (layer B.Cu) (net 2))
 (segment (start 96.393 91.694) (end 96.393 93.599) (width 0.75) (layer B.Cu) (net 2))
 (segment (start 96.393 93.599) (end 97.79 94.996) (width 0.75) (layer B.Cu) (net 2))
 (segment (start 97.79 94.996) (end 100.584 94.996) (width 0.75) (layer B.Cu) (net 2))
 (segment (start 100.584 94.996) (end 103.378 92.202) (width 0.75) (layer B.Cu) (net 2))
 (segment (start 107.352 92.202) (end 109.76699 89.78701) (width 0.75) (layer B.Cu) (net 2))
 (segment (start 106.553 92.202) (end 107.352 92.202) (width 0.75) (layer B.Cu) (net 2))
 (segment (start 103.378 92.202) (end 106.553 92.202) (width 0.75) (layer B.Cu) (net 2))
 (segment (start 109.76699 89.78701) (end 109.76699 89.662) (width 0.75) (layer B.Cu) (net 2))
 (segment (start 109.76699 87.24701) (end 109.76699 87.122) (width 0.75) (layer B.Cu) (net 2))
 (segment (start 107.315 89.699) (end 109.76699 87.24701) (width 0.75) (layer B.Cu) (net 2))
 (segment (start 107.315 92.202) (end 107.315 89.699) (width 0.75) (layer B.Cu) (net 2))
 (segment (start 106.553 92.202) (end 107.315 92.202) (width 0.75) (layer B.Cu) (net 2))
 (segment (start 107.315 92.202) (end 109.76699 92.202) (width 0.75) (layer B.Cu) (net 2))
 (segment (start 104.77301 82.38401) (end 104.648 82.38401) (width 0.75) (layer B.Cu) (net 2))
 (segment (start 107.315 89.699) (end 107.315 84.926) (width 0.75) (layer B.Cu) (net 2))
 (segment (start 106.9525 84.5635) (end 106.9525 78.5945) (width 0.75) (layer B.Cu) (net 2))
 (segment (start 107.315 84.926) (end 106.9525 84.5635) (width 0.75) (layer B.Cu) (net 2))
 (segment (start 106.9525 84.5635) (end 104.77301 82.38401) (width 0.75) (layer B.Cu) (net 2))
 (segment (start 108.331 77.216) (end 108.331 72.644) (width 0.75) (layer B.Cu) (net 2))
 (segment (start 106.9525 78.5945) (end 108.331 77.216) (width 0.75) (layer B.Cu) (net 2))
 (segment (start 104.648 80.809) (end 104.648 76.708) (width 0.75) (layer B.Cu) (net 10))
 (segment (start 84.782901 93.779099) (end 86.179901 93.779099) (width 0.75) (layer F.Cu) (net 1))
 (segment (start 83.82 94.742) (end 84.782901 93.779099) (width 0.75) (layer F.Cu) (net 1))
 (segment (start 89.281 90.678) (end 91.186 90.678) (width 0.75) (layer F.Cu) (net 1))
 (segment (start 86.179901 93.779099) (end 89.281 90.678) (width 0.75) (layer F.Cu) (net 1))
 (segment (start 91.186 90.678) (end 92.71 92.202) (width 0.75) (layer F.Cu) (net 1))
 (segment (start 92.71 96.2152) (end 92.6592 96.266) (width 0.75) (layer F.Cu) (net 1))
 (segment (start 92.71 92.202) (end 92.71 96.2152) (width 0.75) (layer F.Cu) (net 1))
 (segment (start 89.281 85.471) (end 92.329 85.471) (width 0.5) (layer F.Cu) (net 11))
 (segment (start 92.329 85.471) (end 94.615 83.185) (width 0.5) (layer F.Cu) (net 11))
 (segment (start 81.915 78.105) (end 89.281 85.471) (width 0.5) (layer F.Cu) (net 11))
 (segment (start 92.075 83.185) (end 89.916 83.185) (width 0.5) (layer F.Cu) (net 12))
 (via (at 84.582 77.216) (size 1.2) (drill 0.6) (layers F.Cu B.Cu) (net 12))
 (segment (start 84.582 77.851) (end 84.582 77.216) (width 0.5) (layer F.Cu) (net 12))
 (segment (start 89.916 83.185) (end 84.582 77.851) (width 0.5) (layer F.Cu) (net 12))
 (segment (start 84.582 73.902) (end 81.915 71.235) (width 0.5) (layer B.Cu) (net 12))
 (segment (start 84.582 77.216) (end 84.582 73.902) (width 0.5) (layer B.Cu) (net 12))
 (segment (start 111.342 87.122) (end 114.3 87.122) (width 0.75) (layer B.Cu) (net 6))
 (segment (start 111.342 89.662) (end 114.3 89.662) (width 0.75) (layer B.Cu) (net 5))
 (segment (start 111.342 92.202) (end 114.3 92.202) (width 0.75) (layer B.Cu) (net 4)))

